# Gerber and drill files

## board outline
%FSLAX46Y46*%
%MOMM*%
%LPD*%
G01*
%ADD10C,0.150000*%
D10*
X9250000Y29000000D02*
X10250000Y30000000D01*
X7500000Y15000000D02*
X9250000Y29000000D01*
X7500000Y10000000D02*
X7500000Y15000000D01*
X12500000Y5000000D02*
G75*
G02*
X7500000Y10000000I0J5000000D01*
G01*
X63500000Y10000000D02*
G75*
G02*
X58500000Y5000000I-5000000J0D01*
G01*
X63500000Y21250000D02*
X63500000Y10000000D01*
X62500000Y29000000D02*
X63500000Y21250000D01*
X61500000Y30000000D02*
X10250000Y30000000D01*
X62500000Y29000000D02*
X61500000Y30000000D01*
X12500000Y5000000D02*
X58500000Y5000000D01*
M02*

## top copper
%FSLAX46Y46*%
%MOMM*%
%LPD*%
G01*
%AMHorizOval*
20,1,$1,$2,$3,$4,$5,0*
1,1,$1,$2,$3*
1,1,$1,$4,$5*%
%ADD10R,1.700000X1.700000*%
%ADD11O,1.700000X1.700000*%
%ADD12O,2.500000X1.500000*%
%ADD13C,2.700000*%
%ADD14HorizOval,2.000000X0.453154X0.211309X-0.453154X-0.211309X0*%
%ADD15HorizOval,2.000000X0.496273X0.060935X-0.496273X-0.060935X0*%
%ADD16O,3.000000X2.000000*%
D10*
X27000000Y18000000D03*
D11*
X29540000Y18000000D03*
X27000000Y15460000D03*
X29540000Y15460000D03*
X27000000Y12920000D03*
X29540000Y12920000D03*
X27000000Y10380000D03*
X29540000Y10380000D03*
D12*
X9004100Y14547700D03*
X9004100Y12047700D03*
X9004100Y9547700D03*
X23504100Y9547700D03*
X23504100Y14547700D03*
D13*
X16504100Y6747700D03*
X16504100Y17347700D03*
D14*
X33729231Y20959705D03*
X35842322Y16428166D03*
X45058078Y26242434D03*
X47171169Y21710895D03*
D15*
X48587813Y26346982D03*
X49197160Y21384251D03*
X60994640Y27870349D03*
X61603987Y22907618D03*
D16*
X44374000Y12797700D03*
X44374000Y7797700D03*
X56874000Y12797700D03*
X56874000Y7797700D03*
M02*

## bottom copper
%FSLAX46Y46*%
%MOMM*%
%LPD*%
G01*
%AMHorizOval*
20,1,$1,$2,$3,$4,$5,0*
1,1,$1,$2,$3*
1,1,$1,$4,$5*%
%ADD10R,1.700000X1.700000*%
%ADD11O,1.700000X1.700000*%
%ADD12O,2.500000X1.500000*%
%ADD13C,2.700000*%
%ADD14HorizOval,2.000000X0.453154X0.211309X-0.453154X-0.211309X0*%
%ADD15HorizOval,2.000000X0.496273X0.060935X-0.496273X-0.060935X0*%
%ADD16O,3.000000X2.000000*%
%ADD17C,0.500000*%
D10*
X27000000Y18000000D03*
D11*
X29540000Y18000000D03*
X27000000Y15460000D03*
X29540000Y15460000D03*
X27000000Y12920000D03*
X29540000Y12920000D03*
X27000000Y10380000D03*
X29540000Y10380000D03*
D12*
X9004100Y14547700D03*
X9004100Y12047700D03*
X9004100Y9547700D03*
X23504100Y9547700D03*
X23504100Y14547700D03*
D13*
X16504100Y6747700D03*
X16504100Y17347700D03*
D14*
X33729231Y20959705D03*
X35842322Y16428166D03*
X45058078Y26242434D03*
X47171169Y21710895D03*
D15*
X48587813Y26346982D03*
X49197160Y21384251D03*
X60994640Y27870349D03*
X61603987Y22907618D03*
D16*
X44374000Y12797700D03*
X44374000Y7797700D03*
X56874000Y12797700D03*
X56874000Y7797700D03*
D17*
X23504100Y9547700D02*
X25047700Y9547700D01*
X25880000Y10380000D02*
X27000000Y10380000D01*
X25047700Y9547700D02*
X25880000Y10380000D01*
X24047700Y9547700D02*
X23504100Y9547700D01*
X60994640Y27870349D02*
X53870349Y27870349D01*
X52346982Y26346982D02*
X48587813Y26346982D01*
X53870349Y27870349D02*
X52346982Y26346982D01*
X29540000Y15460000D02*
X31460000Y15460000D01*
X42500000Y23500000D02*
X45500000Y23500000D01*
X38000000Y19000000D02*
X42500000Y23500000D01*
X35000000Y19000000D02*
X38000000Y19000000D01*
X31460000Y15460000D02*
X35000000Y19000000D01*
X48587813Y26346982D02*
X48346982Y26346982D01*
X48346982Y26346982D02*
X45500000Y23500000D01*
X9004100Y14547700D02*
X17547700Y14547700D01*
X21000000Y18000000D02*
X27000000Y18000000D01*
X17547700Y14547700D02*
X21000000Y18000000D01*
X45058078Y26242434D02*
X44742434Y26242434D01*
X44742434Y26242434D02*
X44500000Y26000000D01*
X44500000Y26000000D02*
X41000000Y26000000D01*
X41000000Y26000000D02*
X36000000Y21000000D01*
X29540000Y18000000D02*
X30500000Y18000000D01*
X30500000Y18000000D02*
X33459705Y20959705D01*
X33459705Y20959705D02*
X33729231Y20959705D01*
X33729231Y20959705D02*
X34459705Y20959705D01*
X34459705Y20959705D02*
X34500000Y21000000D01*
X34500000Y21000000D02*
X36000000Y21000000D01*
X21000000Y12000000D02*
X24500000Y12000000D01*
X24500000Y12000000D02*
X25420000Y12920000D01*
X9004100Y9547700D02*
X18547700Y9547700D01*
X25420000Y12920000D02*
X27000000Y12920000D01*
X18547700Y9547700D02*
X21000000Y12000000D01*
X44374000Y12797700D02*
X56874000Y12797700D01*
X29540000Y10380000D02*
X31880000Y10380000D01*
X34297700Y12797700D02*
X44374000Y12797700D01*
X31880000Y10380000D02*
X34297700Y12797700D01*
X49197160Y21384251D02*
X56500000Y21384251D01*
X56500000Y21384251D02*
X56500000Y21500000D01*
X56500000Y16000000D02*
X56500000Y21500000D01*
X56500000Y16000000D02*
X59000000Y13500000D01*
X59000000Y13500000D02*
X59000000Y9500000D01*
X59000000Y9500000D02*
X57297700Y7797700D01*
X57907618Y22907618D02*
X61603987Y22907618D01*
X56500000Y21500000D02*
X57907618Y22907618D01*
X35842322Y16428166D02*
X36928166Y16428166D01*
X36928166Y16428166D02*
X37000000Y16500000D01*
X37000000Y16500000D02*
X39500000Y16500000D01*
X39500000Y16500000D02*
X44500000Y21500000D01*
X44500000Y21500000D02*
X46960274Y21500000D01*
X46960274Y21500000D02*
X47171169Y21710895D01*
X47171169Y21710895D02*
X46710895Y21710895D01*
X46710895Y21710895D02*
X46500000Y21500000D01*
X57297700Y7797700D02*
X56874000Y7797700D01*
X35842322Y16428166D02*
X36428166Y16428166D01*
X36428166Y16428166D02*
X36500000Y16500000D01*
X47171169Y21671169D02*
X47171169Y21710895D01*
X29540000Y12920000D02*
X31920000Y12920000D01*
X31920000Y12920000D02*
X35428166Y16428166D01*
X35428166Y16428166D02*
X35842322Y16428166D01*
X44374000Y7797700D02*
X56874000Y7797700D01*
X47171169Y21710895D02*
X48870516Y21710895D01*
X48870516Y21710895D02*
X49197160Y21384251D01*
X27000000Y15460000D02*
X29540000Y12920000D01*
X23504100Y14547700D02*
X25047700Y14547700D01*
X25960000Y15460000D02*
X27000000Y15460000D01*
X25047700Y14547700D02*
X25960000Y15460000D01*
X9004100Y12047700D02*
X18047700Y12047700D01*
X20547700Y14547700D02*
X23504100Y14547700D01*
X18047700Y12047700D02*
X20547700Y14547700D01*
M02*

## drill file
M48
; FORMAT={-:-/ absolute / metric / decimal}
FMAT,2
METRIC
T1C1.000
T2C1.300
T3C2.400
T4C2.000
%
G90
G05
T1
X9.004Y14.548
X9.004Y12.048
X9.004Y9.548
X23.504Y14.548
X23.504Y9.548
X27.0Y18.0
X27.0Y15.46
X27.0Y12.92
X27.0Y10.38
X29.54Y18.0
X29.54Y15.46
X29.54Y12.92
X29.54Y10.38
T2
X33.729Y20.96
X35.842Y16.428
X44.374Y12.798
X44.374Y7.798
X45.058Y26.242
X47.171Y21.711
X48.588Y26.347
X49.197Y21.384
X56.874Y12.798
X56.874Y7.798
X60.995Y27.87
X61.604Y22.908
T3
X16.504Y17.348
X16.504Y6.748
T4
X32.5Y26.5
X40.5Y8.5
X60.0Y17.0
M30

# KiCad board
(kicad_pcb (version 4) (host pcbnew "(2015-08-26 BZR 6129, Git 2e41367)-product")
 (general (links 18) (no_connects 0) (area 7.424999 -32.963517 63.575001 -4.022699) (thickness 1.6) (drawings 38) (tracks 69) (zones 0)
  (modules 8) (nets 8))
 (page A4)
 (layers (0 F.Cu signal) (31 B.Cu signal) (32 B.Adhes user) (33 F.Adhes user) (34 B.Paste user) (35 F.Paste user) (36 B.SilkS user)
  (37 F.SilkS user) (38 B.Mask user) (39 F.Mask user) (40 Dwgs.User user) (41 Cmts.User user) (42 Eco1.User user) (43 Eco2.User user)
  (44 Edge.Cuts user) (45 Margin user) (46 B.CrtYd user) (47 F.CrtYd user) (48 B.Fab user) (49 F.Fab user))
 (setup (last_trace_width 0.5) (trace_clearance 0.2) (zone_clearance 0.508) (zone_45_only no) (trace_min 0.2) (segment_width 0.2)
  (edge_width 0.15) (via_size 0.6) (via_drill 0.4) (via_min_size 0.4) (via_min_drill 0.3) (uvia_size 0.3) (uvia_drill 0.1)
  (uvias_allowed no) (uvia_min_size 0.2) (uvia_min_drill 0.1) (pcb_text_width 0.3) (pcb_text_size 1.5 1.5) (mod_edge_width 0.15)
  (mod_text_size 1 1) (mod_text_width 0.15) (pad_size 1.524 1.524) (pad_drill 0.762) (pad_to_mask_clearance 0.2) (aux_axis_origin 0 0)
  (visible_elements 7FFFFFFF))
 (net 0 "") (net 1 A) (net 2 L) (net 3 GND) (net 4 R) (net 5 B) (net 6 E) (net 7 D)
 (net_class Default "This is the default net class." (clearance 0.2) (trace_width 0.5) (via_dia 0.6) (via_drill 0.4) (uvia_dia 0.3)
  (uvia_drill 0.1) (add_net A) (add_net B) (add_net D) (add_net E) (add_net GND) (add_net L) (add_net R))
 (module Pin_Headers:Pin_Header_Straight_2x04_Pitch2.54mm (layer F.Cu) (at 27 -18)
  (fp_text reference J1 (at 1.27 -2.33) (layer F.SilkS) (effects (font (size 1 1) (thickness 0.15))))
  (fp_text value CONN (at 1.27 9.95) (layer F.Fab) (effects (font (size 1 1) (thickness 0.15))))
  (pad 1 thru_hole rect (at 0 0) (size 1.7 1.7) (drill 1) (layers *.Cu *.Mask) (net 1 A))
  (pad 2 thru_hole oval (at 2.54 0) (size 1.7 1.7) (drill 1) (layers *.Cu *.Mask) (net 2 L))
  (pad 3 thru_hole oval (at 0 2.54) (size 1.7 1.7) (drill 1) (layers *.Cu *.Mask) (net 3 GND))
  (pad 4 thru_hole oval (at 2.54 2.54) (size 1.7 1.7) (drill 1) (layers *.Cu *.Mask) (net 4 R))
  (pad 5 thru_hole oval (at 0 5.08) (size 1.7 1.7) (drill 1) (layers *.Cu *.Mask) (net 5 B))
  (pad 6 thru_hole oval (at 2.54 5.08) (size 1.7 1.7) (drill 1) (layers *.Cu *.Mask) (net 3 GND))
  (pad 7 thru_hole oval (at 0 7.62) (size 1.7 1.7) (drill 1) (layers *.Cu *.Mask) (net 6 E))
  (pad 8 thru_hole oval (at 2.54 7.62) (size 1.7 1.7) (drill 1) (layers *.Cu *.Mask) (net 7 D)))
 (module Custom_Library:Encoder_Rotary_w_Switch (layer F.Cu) (at 16.5041 -12.0477)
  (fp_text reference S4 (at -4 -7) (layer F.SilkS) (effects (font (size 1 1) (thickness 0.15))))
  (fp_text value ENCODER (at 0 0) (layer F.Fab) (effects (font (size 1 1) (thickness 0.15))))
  (pad 1 thru_hole oval (at -7.5 -2.5) (size 2.5 1.5) (drill 1) (layers *.Cu *.Mask F.SilkS) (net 1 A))
  (pad 2 thru_hole oval (at -7.5 0) (size 2.5 1.5) (drill 1) (layers *.Cu *.Mask F.SilkS) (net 3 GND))
  (pad 3 thru_hole oval (at -7.5 2.5) (size 2.5 1.5) (drill 1) (layers *.Cu *.Mask F.SilkS) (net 5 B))
  (pad 4 thru_hole oval (at 7 2.5) (size 2.5 1.5) (drill 1) (layers *.Cu *.Mask F.SilkS) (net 6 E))
  (pad 5 thru_hole oval (at 7 -2.5) (size 2.5 1.5) (drill 1) (layers *.Cu *.Mask F.SilkS) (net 3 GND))
  (pad "" thru_hole circle (at 0 5.3) (size 2.7 2.7) (drill 2.4) (layers *.Cu *.Mask F.SilkS))
  (pad "" thru_hole circle (at 0 -5.3) (size 2.7 2.7) (drill 2.4) (layers *.Cu *.Mask F.SilkS)))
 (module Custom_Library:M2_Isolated (layer F.Cu) (at 32.5 -26.5)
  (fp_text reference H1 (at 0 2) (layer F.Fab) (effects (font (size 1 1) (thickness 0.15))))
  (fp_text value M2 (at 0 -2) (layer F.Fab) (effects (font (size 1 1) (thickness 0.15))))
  (pad "" np_thru_hole circle (at 0 0) (size 2 2) (drill 2) (layers *.Cu *.Mask F.SilkS) (solder_mask_margin 1.5) (clearance 1.7)))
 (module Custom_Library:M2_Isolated (layer F.Cu) (at 40.5 -8.5)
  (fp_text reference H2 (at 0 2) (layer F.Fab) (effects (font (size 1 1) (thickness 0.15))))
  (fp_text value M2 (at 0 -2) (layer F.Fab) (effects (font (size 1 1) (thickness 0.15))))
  (pad "" np_thru_hole circle (at 0 0) (size 2 2) (drill 2) (layers *.Cu *.Mask F.SilkS) (solder_mask_margin 1.5) (clearance 1.7)))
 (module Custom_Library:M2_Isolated (layer F.Cu) (at 60 -17)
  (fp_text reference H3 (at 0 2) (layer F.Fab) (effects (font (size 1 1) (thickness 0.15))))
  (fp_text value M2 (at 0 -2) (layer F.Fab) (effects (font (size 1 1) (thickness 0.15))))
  (pad "" np_thru_hole circle (at 0 0) (size 2 2) (drill 2) (layers *.Cu *.Mask F.SilkS) (solder_mask_margin 1.5) (clearance 1.7)))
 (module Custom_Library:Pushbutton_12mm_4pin (layer F.Cu) (at 40.4502 -21.3353 25)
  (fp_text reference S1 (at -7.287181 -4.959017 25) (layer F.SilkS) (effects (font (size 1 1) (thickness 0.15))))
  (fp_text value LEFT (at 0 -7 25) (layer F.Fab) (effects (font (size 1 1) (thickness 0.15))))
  (pad 1 thru_hole oval (at -6.25 -2.5 25) (size 3 2) (drill 1.3) (layers *.Cu *.Mask F.SilkS) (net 2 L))
  (pad 2 thru_hole oval (at -6.25 2.5 25) (size 3 2) (drill 1.3) (layers *.Cu *.Mask F.SilkS) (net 3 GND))
  (pad 1 thru_hole oval (at 6.25 -2.5 25) (size 3 2) (drill 1.3) (layers *.Cu *.Mask F.SilkS) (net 2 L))
  (pad 2 thru_hole oval (at 6.25 2.5 25) (size 3 2) (drill 1.3) (layers *.Cu *.Mask F.SilkS) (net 3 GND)))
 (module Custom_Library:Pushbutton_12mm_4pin (layer F.Cu) (at 55.0959 -24.6273 7)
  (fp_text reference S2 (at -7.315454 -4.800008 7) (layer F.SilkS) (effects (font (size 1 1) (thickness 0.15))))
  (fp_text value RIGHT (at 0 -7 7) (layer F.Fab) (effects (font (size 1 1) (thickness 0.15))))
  (pad 1 thru_hole oval (at -6.25 -2.5 7) (size 3 2) (drill 1.3) (layers *.Cu *.Mask F.SilkS) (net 4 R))
  (pad 2 thru_hole oval (at -6.25 2.5 7) (size 3 2) (drill 1.3) (layers *.Cu *.Mask F.SilkS) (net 3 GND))
  (pad 1 thru_hole oval (at 6.25 -2.5 7) (size 3 2) (drill 1.3) (layers *.Cu *.Mask F.SilkS) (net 4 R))
  (pad 2 thru_hole oval (at 6.25 2.5 7) (size 3 2) (drill 1.3) (layers *.Cu *.Mask F.SilkS) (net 3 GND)))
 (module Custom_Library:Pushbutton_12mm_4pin (layer F.Cu) (at 50.624 -10.2977)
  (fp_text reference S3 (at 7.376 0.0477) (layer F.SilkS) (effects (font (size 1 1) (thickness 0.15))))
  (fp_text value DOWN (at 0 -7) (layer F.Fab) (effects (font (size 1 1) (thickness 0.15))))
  (pad 1 thru_hole oval (at -6.25 -2.5) (size 3 2) (drill 1.3) (layers *.Cu *.Mask F.SilkS) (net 7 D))
  (pad 2 thru_hole oval (at -6.25 2.5) (size 3 2) (drill 1.3) (layers *.Cu *.Mask F.SilkS) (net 3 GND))
  (pad 1 thru_hole oval (at 6.25 -2.5) (size 3 2) (drill 1.3) (layers *.Cu *.Mask F.SilkS) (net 7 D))
  (pad 2 thru_hole oval (at 6.25 2.5) (size 3 2) (drill 1.3) (layers *.Cu *.Mask F.SilkS) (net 3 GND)))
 (gr_line (start 9.25 -29) (end 10.25 -30) (angle 90) (layer Edge.Cuts) (width 0.15))
 (gr_line (start 7.5 -15) (end 9.25 -29) (angle 90) (layer Edge.Cuts) (width 0.15))
 (gr_line (start 7.5 -10) (end 7.5 -15) (angle 90) (layer Edge.Cuts) (width 0.15))
 (gr_arc (start 12.5 -10) (end 12.5 -5) (angle 90) (layer Edge.Cuts) (width 0.15))
 (gr_arc (start 58.5 -10) (end 63.5 -10) (angle 90) (layer Edge.Cuts) (width 0.15))
 (gr_line (start 63.5 -21.25) (end 63.5 -10) (angle 90) (layer Edge.Cuts) (width 0.15))
 (gr_line (start 62.5 -29) (end 63.5 -21.25) (angle 90) (layer Edge.Cuts) (width 0.15))
 (gr_line (start 61.5 -30) (end 10.25 -30) (angle 90) (layer Edge.Cuts) (width 0.15))
 (gr_line (start 62.5 -29) (end 61.5 -30) (angle 90) (layer Edge.Cuts) (width 0.15))
 (gr_line (start 12.5 -5) (end 58.5 -5) (angle 90) (layer Edge.Cuts) (width 0.15))
 (segment (start 23.5041 -9.5477) (end 25.0477 -9.5477) (width 0.5) (layer B.Cu) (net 6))
 (segment (start 25.88 -10.38) (end 27 -10.38) (width 0.5) (layer B.Cu) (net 6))
 (segment (start 25.0477 -9.5477) (end 25.88 -10.38) (width 0.5) (layer B.Cu) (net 6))
 (segment (start 24.0477 -9.5477) (end 23.5041 -9.5477) (width 0.5) (layer B.Cu) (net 6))
 (segment (start 60.99464 -27.870349) (end 53.870349 -27.870349) (width 0.5) (layer B.Cu) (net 4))
 (segment (start 52.346982 -26.346982) (end 48.587813 -26.346982) (width 0.5) (layer B.Cu) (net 4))
 (segment (start 53.870349 -27.870349) (end 52.346982 -26.346982) (width 0.5) (layer B.Cu) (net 4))
 (segment (start 29.54 -15.46) (end 31.46 -15.46) (width 0.5) (layer B.Cu) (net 4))
 (segment (start 42.5 -23.5) (end 45.5 -23.5) (width 0.5) (layer B.Cu) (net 4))
 (segment (start 38 -19) (end 42.5 -23.5) (width 0.5) (layer B.Cu) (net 4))
 (segment (start 35 -19) (end 38 -19) (width 0.5) (layer B.Cu) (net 4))
 (segment (start 31.46 -15.46) (end 35 -19) (width 0.5) (layer B.Cu) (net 4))
 (segment (start 48.587813 -26.346982) (end 48.346982 -26.346982) (width 0.5) (layer B.Cu) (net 4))
 (segment (start 48.346982 -26.346982) (end 45.5 -23.5) (width 0.5) (layer B.Cu) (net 4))
 (segment (start 9.0041 -14.5477) (end 17.5477 -14.5477) (width 0.5) (layer B.Cu) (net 1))
 (segment (start 21 -18) (end 27 -18) (width 0.5) (layer B.Cu) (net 1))
 (segment (start 17.5477 -14.5477) (end 21 -18) (width 0.5) (layer B.Cu) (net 1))
 (segment (start 45.058078 -26.242434) (end 44.742434 -26.242434) (width 0.5) (layer B.Cu) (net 2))
 (segment (start 44.742434 -26.242434) (end 44.5 -26) (width 0.5) (layer B.Cu) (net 2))
 (segment (start 44.5 -26) (end 41 -26) (width 0.5) (layer B.Cu) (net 2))
 (segment (start 41 -26) (end 36 -21) (width 0.5) (layer B.Cu) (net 2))
 (segment (start 29.54 -18) (end 30.5 -18) (width 0.5) (layer B.Cu) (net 2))
 (segment (start 30.5 -18) (end 33.459705 -20.959705) (width 0.5) (layer B.Cu) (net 2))
 (segment (start 33.459705 -20.959705) (end 33.729231 -20.959705) (width 0.5) (layer B.Cu) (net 2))
 (segment (start 33.729231 -20.959705) (end 34.459705 -20.959705) (width 0.5) (layer B.Cu) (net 2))
 (segment (start 34.459705 -20.959705) (end 34.5 -21) (width 0.5) (layer B.Cu) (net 2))
 (segment (start 34.5 -21) (end 36 -21) (width 0.5) (layer B.Cu) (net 2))
 (segment (start 21 -12) (end 24.5 -12) (width 0.5) (layer B.Cu) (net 5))
 (segment (start 24.5 -12) (end 25.42 -12.92) (width 0.5) (layer B.Cu) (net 5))
 (segment (start 9.0041 -9.5477) (end 18.5477 -9.5477) (width 0.5) (layer B.Cu) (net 5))
 (segment (start 25.42 -12.92) (end 27 -12.92) (width 0.5) (layer B.Cu) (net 5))
 (segment (start 18.5477 -9.5477) (end 21 -12) (width 0.5) (layer B.Cu) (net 5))
 (segment (start 44.374 -12.7977) (end 56.874 -12.7977) (width 0.5) (layer B.Cu) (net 7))
 (segment (start 29.54 -10.38) (end 31.88 -10.38) (width 0.5) (layer B.Cu) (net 7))
 (segment (start 34.2977 -12.7977) (end 44.374 -12.7977) (width 0.5) (layer B.Cu) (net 7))
 (segment (start 31.88 -10.38) (end 34.2977 -12.7977) (width 0.5) (layer B.Cu) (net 7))
 (segment (start 49.19716 -21.384251) (end 56.5 -21.384251) (width 0.5) (layer B.Cu) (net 3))
 (segment (start 56.5 -21.384251) (end 56.5 -21.5) (width 0.5) (layer B.Cu) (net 3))
 (segment (start 56.5 -16) (end 56.5 -21.5) (width 0.5) (layer B.Cu) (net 3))
 (segment (start 56.5 -16) (end 59 -13.5) (width 0.5) (layer B.Cu) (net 3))
 (segment (start 59 -13.5) (end 59 -9.5) (width 0.5) (layer B.Cu) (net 3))
 (segment (start 59 -9.5) (end 57.2977 -7.7977) (width 0.5) (layer B.Cu) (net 3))
 (segment (start 57.907618 -22.907618) (end 61.603987 -22.907618) (width 0.5) (layer B.Cu) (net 3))
 (segment (start 56.5 -21.5) (end 57.907618 -22.907618) (width 0.5) (layer B.Cu) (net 3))
 (segment (start 35.842322 -16.428166) (end 36.928166 -16.428166) (width 0.5) (layer B.Cu) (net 3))
 (segment (start 36.928166 -16.428166) (end 37 -16.5) (width 0.5) (layer B.Cu) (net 3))
 (segment (start 37 -16.5) (end 39.5 -16.5) (width 0.5) (layer B.Cu) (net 3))
 (segment (start 39.5 -16.5) (end 44.5 -21.5) (width 0.5) (layer B.Cu) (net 3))
 (segment (start 44.5 -21.5) (end 46.960274 -21.5) (width 0.5) (layer B.Cu) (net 3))
 (segment (start 46.960274 -21.5) (end 47.171169 -21.710895) (width 0.5) (layer B.Cu) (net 3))
 (segment (start 47.171169 -21.710895) (end 46.710895 -21.710895) (width 0.5) (layer B.Cu) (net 3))
 (segment (start 46.710895 -21.710895) (end 46.5 -21.5) (width 0.5) (layer B.Cu) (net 3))
 (segment (start 57.2977 -7.7977) (end 56.874 -7.7977) (width 0.5) (layer B.Cu) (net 3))
 (segment (start 35.842322 -16.428166) (end 36.428166 -16.428166) (width 0.5) (layer B.Cu) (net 3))
 (segment (start 36.428166 -16.428166) (end 36.5 -16.5) (width 0.5) (layer B.Cu) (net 3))
 (segment (start 47.171169 -21.671169) (end 47.171169 -21.710895) (width 0.5) (layer B.Cu) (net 3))
 (segment (start 29.54 -12.92) (end 31.92 -12.92) (width 0.5) (layer B.Cu) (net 3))
 (segment (start 31.92 -12.92) (end 35.428166 -16.428166) (width 0.5) (layer B.Cu) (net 3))
 (segment (start 35.428166 -16.428166) (end 35.842322 -16.428166) (width 0.5) (layer B.Cu) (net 3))
 (segment (start 44.374 -7.7977) (end 56.874 -7.7977) (width 0.5) (layer B.Cu) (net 3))
 (segment (start 47.171169 -21.710895) (end 48.870516 -21.710895) (width 0.5) (layer B.Cu) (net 3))
 (segment (start 48.870516 -21.710895) (end 49.19716 -21.384251) (width 0.5) (layer B.Cu) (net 3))
 (segment (start 27 -15.46) (end 29.54 -12.92) (width 0.5) (layer B.Cu) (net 3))
 (segment (start 23.5041 -14.5477) (end 25.0477 -14.5477) (width 0.5) (layer B.Cu) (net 3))
 (segment (start 25.96 -15.46) (end 27 -15.46) (width 0.5) (layer B.Cu) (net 3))
 (segment (start 25.0477 -14.5477) (end 25.96 -15.46) (width 0.5) (layer B.Cu) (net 3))
 (segment (start 9.0041 -12.0477) (end 18.0477 -12.0477) (width 0.5) (layer B.Cu) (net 3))
 (segment (start 20.5477 -14.5477) (end 23.5041 -14.5477) (width 0.5) (layer B.Cu) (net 3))
 (segment (start 18.0477 -12.0477) (end 20.5477 -14.5477) (width 0.5) (layer B.Cu) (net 3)))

